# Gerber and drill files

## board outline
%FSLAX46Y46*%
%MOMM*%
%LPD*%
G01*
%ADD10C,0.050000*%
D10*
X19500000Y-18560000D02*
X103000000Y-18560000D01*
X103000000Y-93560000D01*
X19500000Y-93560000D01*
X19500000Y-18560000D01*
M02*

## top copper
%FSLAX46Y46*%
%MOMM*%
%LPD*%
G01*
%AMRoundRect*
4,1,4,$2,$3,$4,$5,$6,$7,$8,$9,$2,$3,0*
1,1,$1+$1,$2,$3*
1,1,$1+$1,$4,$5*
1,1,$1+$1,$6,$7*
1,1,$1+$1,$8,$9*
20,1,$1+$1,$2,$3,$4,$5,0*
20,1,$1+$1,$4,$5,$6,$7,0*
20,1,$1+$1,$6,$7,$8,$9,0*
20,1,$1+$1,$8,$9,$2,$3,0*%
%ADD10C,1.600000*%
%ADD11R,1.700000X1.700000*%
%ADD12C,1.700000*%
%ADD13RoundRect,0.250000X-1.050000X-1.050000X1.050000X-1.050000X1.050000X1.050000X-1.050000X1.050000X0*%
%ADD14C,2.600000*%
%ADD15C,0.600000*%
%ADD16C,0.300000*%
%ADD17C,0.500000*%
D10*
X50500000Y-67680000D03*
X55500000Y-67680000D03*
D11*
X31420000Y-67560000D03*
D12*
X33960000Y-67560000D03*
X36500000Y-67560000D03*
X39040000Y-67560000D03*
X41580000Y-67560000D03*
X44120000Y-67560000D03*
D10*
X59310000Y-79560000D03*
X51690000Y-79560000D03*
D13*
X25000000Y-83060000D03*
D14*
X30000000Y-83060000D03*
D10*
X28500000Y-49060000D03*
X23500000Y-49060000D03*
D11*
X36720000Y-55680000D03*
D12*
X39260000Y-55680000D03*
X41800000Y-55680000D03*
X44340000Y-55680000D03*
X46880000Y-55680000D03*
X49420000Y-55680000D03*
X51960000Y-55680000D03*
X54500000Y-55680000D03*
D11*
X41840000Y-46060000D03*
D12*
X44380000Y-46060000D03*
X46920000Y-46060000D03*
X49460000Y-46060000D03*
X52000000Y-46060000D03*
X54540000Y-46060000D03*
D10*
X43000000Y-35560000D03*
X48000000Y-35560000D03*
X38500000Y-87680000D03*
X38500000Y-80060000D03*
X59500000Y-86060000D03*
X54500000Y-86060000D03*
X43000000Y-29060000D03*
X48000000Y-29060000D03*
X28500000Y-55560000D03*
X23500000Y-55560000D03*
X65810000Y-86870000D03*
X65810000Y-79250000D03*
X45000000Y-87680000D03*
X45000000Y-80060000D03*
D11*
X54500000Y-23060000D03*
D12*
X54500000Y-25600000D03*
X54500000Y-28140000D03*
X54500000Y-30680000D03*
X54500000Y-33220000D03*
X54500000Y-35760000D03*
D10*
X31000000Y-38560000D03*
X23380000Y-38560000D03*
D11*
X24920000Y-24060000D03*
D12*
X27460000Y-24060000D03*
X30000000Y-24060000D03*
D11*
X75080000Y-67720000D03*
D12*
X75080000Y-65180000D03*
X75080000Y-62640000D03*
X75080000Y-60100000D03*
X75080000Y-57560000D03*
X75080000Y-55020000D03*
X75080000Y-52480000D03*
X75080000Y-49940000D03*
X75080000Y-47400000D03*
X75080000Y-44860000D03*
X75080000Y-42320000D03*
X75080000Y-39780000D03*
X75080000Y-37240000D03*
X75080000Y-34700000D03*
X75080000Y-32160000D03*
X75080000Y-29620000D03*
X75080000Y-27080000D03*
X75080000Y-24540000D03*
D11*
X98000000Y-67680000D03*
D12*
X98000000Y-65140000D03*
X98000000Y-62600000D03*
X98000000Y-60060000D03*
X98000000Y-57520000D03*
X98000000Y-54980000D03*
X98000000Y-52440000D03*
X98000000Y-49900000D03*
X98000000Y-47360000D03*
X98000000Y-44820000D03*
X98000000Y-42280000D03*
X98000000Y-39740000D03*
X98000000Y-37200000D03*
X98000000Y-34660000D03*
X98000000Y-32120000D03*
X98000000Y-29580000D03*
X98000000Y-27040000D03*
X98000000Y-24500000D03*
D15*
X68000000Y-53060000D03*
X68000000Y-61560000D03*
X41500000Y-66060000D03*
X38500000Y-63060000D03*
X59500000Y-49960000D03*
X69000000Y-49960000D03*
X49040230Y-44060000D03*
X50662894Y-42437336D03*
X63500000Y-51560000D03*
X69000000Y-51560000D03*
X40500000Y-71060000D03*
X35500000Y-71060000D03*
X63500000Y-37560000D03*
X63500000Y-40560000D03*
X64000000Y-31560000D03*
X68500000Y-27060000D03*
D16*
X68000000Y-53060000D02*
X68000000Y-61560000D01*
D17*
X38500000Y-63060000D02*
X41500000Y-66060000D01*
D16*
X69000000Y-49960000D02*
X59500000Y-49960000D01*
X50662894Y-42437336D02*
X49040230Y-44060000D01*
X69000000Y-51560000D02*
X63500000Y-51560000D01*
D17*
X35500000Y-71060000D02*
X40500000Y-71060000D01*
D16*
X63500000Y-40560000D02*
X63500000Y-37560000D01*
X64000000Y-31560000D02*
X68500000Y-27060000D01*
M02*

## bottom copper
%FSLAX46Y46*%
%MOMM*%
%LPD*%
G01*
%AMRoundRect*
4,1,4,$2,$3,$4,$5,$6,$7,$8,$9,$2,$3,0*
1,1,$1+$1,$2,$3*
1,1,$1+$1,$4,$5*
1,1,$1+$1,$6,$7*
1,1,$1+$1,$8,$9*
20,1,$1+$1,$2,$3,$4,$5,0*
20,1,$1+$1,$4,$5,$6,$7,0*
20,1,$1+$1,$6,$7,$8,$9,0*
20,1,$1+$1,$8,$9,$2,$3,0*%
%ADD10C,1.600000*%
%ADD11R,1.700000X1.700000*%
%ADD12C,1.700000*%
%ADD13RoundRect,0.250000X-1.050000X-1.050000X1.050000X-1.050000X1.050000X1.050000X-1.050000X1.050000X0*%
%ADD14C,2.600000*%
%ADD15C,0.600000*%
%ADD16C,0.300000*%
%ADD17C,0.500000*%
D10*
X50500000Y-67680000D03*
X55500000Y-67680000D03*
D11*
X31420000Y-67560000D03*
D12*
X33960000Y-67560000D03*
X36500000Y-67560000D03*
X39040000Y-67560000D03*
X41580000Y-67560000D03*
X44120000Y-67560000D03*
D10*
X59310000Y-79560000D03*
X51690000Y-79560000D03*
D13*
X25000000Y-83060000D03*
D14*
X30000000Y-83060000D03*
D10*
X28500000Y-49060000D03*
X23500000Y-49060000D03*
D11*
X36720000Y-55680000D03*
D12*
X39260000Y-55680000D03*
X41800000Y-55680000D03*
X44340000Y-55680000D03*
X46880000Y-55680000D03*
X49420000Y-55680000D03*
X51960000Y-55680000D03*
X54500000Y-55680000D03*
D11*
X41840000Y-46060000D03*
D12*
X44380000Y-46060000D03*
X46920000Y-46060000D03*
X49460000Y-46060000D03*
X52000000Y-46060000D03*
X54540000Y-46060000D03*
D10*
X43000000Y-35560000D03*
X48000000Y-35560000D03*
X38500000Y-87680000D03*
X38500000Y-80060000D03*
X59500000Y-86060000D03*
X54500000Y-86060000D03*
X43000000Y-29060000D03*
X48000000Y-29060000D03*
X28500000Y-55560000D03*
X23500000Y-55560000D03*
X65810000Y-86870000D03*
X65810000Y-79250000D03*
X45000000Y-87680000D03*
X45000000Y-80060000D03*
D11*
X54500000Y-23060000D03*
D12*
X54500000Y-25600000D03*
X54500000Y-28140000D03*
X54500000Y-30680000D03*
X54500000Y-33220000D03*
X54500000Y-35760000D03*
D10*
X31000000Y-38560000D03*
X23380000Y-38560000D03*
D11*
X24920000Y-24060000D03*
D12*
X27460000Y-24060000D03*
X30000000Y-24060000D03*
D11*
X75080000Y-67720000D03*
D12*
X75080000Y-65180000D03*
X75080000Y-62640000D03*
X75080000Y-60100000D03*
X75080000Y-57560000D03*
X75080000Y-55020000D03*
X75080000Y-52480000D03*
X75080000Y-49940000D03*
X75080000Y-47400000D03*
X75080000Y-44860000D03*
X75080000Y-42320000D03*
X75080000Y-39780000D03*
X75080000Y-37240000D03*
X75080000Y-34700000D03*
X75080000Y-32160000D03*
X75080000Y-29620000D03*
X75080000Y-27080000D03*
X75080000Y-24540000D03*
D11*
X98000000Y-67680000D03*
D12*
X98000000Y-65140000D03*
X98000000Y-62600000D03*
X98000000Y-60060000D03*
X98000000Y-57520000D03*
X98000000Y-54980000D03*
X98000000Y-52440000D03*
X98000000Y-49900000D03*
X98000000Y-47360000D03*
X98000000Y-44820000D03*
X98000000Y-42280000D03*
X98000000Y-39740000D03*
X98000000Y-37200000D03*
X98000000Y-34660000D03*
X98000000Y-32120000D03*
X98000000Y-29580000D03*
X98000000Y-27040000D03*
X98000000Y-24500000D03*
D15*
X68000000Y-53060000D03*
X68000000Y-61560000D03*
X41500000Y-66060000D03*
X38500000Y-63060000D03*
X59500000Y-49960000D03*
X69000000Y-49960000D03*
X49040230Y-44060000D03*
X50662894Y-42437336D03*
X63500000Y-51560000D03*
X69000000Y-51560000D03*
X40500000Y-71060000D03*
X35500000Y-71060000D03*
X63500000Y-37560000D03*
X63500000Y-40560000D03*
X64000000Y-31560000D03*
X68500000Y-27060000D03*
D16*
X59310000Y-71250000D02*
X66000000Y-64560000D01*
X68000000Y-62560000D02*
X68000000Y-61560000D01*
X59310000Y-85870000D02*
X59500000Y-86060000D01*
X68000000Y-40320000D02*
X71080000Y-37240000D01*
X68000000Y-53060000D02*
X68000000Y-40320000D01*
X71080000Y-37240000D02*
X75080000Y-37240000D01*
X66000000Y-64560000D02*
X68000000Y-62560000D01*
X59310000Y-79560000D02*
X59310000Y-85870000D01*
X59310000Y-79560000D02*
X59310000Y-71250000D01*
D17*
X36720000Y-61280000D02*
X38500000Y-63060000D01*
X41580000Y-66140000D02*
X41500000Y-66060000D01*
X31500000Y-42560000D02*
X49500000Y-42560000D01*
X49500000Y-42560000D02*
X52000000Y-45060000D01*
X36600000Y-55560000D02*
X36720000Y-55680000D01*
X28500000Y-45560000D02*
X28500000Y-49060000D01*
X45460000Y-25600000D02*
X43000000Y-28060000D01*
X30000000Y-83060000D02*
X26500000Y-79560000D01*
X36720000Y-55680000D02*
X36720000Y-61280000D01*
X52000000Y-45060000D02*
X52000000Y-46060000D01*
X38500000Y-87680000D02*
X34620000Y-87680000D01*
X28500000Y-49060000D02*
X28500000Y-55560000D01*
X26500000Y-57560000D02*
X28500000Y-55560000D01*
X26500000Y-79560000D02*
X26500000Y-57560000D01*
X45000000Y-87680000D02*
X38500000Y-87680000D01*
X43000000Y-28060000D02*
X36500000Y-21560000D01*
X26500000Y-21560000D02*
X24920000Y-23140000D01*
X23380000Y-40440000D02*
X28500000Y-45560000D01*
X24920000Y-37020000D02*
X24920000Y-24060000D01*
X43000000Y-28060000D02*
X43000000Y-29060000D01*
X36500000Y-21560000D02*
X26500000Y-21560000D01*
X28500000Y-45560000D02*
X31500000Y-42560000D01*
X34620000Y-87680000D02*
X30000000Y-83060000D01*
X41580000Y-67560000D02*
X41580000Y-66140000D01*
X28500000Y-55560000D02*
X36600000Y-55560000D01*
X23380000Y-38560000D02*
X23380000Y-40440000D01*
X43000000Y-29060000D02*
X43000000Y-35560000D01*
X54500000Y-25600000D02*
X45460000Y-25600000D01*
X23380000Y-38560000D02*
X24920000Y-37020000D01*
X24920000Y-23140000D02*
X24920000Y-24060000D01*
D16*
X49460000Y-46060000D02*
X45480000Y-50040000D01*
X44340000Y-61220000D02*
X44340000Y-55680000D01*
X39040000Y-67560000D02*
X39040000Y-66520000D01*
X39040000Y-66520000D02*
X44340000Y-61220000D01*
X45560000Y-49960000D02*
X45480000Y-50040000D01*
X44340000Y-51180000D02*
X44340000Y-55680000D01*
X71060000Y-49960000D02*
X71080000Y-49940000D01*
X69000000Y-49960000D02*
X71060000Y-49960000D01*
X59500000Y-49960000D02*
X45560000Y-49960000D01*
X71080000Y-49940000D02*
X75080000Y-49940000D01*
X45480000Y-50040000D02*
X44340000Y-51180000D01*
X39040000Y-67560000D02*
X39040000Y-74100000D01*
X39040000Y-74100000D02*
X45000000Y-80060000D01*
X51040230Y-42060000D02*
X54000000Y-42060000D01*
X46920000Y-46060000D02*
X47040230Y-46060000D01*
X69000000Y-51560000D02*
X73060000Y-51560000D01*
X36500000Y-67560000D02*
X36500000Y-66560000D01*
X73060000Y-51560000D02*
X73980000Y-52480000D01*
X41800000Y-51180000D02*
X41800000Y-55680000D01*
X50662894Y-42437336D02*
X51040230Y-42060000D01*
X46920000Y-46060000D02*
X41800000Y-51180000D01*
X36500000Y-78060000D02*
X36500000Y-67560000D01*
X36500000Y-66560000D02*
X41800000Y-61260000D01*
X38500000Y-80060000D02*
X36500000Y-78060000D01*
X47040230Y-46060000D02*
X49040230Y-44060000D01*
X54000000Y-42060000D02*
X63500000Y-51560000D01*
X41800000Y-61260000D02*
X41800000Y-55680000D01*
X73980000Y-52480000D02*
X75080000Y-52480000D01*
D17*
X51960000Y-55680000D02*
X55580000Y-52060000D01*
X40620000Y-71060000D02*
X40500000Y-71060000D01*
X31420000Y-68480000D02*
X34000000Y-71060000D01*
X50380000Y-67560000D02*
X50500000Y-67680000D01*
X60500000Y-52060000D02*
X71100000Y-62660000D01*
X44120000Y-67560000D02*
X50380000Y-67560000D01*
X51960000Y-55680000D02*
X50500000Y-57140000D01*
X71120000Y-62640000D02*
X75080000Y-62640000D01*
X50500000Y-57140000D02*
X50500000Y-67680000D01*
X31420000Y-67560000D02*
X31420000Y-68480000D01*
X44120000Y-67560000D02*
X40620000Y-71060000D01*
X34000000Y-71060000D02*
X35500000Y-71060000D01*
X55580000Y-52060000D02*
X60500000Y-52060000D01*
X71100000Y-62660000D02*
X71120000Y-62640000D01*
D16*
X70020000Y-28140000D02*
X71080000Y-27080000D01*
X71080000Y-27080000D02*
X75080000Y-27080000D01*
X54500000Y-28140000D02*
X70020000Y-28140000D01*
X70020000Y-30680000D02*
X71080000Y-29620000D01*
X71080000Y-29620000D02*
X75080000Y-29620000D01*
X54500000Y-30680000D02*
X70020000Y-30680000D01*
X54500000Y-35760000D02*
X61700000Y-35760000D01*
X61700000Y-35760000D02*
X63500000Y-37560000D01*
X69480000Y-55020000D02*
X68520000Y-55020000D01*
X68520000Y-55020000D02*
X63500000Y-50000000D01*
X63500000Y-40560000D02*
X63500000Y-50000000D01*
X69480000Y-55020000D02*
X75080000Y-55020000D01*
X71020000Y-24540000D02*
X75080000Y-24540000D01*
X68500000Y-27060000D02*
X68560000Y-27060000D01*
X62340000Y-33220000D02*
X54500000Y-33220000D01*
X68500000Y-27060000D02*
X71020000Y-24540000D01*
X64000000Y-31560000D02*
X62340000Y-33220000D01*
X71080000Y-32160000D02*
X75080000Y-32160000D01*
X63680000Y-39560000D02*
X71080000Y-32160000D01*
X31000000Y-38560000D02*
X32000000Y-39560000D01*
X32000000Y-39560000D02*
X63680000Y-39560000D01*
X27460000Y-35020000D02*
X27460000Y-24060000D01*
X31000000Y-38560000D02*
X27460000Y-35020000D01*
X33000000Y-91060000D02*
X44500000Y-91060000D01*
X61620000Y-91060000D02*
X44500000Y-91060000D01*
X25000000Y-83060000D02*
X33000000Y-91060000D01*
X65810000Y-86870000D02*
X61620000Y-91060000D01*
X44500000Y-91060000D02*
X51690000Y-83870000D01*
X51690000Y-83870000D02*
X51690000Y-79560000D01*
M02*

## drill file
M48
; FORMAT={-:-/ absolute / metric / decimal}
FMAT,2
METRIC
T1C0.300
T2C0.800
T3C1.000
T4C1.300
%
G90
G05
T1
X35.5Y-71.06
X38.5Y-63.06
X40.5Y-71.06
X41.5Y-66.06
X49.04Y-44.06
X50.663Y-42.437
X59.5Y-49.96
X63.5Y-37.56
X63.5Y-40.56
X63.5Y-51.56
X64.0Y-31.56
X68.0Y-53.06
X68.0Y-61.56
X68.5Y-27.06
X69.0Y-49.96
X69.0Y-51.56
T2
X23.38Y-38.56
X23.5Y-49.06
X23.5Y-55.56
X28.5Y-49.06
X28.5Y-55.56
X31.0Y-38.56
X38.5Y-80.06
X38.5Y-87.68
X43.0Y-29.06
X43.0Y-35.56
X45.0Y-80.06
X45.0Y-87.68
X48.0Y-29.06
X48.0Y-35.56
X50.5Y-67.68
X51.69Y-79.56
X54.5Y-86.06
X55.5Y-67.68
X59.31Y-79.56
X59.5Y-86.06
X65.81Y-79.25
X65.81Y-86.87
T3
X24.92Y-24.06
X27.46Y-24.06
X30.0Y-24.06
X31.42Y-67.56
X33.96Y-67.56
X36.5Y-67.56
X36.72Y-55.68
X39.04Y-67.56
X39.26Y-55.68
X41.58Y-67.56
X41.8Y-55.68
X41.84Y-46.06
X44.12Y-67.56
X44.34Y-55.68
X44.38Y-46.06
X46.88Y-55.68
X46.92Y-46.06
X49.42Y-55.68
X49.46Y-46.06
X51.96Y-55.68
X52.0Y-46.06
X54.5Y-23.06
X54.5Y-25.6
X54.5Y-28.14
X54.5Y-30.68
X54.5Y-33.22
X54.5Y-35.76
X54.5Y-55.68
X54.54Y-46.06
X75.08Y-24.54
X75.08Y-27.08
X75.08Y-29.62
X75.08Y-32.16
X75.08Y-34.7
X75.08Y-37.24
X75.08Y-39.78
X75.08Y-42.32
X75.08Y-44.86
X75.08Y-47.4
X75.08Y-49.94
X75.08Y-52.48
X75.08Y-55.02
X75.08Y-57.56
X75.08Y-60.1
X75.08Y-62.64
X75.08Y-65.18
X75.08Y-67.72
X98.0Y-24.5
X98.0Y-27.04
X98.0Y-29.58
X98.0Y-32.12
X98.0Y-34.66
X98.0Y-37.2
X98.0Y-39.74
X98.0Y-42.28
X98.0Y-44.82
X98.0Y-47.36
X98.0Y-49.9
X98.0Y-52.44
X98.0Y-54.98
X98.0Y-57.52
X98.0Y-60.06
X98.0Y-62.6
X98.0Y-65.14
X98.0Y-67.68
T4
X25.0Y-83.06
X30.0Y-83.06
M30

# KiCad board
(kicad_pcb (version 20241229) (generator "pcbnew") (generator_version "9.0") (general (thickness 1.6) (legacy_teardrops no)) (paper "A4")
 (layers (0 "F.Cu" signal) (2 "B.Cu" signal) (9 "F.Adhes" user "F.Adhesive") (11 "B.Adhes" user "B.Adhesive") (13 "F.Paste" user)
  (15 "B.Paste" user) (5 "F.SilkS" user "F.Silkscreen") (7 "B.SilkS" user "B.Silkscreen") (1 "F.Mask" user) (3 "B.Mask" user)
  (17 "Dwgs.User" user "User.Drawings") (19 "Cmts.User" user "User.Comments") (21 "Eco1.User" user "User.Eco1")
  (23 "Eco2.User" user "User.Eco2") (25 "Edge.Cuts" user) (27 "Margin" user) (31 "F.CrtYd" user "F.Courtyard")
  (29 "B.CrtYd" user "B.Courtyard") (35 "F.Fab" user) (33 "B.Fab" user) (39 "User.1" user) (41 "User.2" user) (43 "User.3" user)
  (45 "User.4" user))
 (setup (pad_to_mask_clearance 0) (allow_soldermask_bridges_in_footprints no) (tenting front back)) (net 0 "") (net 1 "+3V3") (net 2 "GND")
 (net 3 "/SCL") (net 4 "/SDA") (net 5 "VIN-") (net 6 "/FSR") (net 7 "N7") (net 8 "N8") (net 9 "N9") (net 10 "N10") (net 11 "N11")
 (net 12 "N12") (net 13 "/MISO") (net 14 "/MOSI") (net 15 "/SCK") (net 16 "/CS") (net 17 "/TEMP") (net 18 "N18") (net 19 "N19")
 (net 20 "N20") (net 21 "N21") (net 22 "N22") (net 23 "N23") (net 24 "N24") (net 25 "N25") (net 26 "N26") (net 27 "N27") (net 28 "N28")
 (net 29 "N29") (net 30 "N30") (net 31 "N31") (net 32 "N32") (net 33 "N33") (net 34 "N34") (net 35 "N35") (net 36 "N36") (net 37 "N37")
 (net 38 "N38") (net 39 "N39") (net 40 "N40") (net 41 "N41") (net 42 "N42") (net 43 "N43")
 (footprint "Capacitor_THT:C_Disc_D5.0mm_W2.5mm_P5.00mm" (layer "F.Cu") (at 50.5 67.68)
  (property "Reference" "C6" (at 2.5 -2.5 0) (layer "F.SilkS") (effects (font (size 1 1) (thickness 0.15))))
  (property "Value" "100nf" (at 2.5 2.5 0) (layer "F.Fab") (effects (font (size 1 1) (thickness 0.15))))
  (pad "1" thru_hole circle (at 0 0) (size 1.6 1.6) (drill 0.8) (layers "*.Cu" "*.Mask") (remove_unused_layers no) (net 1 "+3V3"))
  (pad "2" thru_hole circle (at 5 0) (size 1.6 1.6) (drill 0.8) (layers "*.Cu" "*.Mask") (remove_unused_layers no) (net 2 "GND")))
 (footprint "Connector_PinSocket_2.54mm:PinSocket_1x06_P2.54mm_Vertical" (layer "F.Cu") (at 31.42 67.56 90)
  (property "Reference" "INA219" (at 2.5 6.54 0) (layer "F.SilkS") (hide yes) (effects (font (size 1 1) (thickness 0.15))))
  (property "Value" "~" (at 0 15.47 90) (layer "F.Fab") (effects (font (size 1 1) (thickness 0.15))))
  (pad "1" thru_hole rect (at 0 0 90) (size 1.7 1.7) (drill 1) (layers "*.Cu" "*.Mask") (remove_unused_layers no) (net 1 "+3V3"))
  (pad "2" thru_hole circle (at 0 2.54 90) (size 1.7 1.7) (drill 1) (layers "*.Cu" "*.Mask") (remove_unused_layers no) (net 2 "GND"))
  (pad "3" thru_hole circle (at 0 5.08 90) (size 1.7 1.7) (drill 1) (layers "*.Cu" "*.Mask") (remove_unused_layers no) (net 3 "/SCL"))
  (pad "4" thru_hole circle (at 0 7.62 90) (size 1.7 1.7) (drill 1) (layers "*.Cu" "*.Mask") (remove_unused_layers no) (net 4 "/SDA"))
  (pad "5" thru_hole circle (at 0 10.16 90) (size 1.7 1.7) (drill 1) (layers "*.Cu" "*.Mask") (remove_unused_layers no) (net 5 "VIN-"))
  (pad "6" thru_hole circle (at 0 12.7 90) (size 1.7 1.7) (drill 1) (layers "*.Cu" "*.Mask") (remove_unused_layers no) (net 1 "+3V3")))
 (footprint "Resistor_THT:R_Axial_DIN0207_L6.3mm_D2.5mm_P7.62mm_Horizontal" (layer "F.Cu") (at 59.31 79.56 180)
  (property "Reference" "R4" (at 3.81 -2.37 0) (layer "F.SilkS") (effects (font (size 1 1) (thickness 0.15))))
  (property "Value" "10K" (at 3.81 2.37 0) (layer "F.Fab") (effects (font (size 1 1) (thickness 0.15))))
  (pad "1" thru_hole circle (at 0 0 180) (size 1.6 1.6) (drill 0.8) (layers "*.Cu" "*.Mask") (remove_unused_layers no) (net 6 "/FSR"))
  (pad "2" thru_hole circle (at 7.62 0 180) (size 1.6 1.6) (drill 0.8) (layers "*.Cu" "*.Mask") (remove_unused_layers no) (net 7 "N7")))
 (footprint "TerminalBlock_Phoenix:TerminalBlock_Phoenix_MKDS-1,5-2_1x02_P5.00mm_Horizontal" (layer "F.Cu") (at 25 83.06)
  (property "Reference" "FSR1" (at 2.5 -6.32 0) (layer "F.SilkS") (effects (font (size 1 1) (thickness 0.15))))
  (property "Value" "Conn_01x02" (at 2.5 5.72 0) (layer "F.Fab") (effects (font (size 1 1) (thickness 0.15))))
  (pad "1" thru_hole roundrect (at 0 0) (size 2.6 2.6) (drill 1.3) (layers "*.Cu" "*.Mask") (remove_unused_layers no)
   (roundrect_rratio 0.096154) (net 7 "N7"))
  (pad "2" thru_hole circle (at 5 0) (size 2.6 2.6) (drill 1.3) (layers "*.Cu" "*.Mask") (remove_unused_layers no) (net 5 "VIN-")))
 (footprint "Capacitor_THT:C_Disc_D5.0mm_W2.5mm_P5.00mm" (layer "F.Cu") (at 28.5 49.06 180)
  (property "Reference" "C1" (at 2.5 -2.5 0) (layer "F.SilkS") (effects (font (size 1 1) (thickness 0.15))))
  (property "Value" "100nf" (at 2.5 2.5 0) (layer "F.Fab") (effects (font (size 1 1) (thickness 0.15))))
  (pad "1" thru_hole circle (at 0 0 180) (size 1.6 1.6) (drill 0.8) (layers "*.Cu" "*.Mask") (remove_unused_layers no) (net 5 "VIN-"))
  (pad "2" thru_hole circle (at 5 0 180) (size 1.6 1.6) (drill 0.8) (layers "*.Cu" "*.Mask") (remove_unused_layers no) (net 2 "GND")))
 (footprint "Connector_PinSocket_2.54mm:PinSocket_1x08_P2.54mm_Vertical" (layer "F.Cu") (at 36.72 55.68 90)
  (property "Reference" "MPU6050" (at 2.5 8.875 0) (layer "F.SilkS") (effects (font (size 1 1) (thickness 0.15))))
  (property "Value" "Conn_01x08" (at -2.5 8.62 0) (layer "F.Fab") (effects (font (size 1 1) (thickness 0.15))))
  (pad "1" thru_hole rect (at 0 0 90) (size 1.7 1.7) (drill 1) (layers "*.Cu" "*.Mask") (remove_unused_layers no) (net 5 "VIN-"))
  (pad "2" thru_hole circle (at 0 2.54 90) (size 1.7 1.7) (drill 1) (layers "*.Cu" "*.Mask") (remove_unused_layers no) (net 2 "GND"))
  (pad "3" thru_hole circle (at 0 5.08 90) (size 1.7 1.7) (drill 1) (layers "*.Cu" "*.Mask") (remove_unused_layers no) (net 3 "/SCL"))
  (pad "4" thru_hole circle (at 0 7.62 90) (size 1.7 1.7) (drill 1) (layers "*.Cu" "*.Mask") (remove_unused_layers no) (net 4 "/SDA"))
  (pad "5" thru_hole circle (at 0 10.16 90) (size 1.7 1.7) (drill 1) (layers "*.Cu" "*.Mask") (remove_unused_layers no) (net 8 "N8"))
  (pad "6" thru_hole circle (at 0 12.7 90) (size 1.7 1.7) (drill 1) (layers "*.Cu" "*.Mask") (remove_unused_layers no) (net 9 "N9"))
  (pad "7" thru_hole circle (at 0 15.24 90) (size 1.7 1.7) (drill 1) (layers "*.Cu" "*.Mask") (remove_unused_layers no) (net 1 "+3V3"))
  (pad "8" thru_hole circle (at 0 17.78 90) (size 1.7 1.7) (drill 1) (layers "*.Cu" "*.Mask") (remove_unused_layers no) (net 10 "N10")))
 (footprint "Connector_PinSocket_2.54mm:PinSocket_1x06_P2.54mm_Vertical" (layer "F.Cu") (at 41.84 46.06 90)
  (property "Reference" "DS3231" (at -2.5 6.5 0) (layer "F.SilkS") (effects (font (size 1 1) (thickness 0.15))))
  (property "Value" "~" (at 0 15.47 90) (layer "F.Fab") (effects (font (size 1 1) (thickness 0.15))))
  (pad "1" thru_hole rect (at 0 0 90) (size 1.7 1.7) (drill 1) (layers "*.Cu" "*.Mask") (remove_unused_layers no) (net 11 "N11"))
  (pad "2" thru_hole circle (at 0 2.54 90) (size 1.7 1.7) (drill 1) (layers "*.Cu" "*.Mask") (remove_unused_layers no) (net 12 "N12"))
  (pad "3" thru_hole circle (at 0 5.08 90) (size 1.7 1.7) (drill 1) (layers "*.Cu" "*.Mask") (remove_unused_layers no) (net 3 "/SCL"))
  (pad "4" thru_hole circle (at 0 7.62 90) (size 1.7 1.7) (drill 1) (layers "*.Cu" "*.Mask") (remove_unused_layers no) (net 4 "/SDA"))
  (pad "5" thru_hole circle (at 0 10.16 90) (size 1.7 1.7) (drill 1) (layers "*.Cu" "*.Mask") (remove_unused_layers no) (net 5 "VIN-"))
  (pad "6" thru_hole circle (at 0 12.7 90) (size 1.7 1.7) (drill 1) (layers "*.Cu" "*.Mask") (remove_unused_layers no) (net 2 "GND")))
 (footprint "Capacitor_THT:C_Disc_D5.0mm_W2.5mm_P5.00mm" (layer "F.Cu") (at 43 35.56)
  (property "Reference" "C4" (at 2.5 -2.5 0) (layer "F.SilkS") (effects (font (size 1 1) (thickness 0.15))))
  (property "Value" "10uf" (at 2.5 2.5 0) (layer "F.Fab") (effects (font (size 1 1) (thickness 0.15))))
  (pad "1" thru_hole circle (at 0 0) (size 1.6 1.6) (drill 0.8) (layers "*.Cu" "*.Mask") (remove_unused_layers no) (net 5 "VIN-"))
  (pad "2" thru_hole circle (at 5 0) (size 1.6 1.6) (drill 0.8) (layers "*.Cu" "*.Mask") (remove_unused_layers no) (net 2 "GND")))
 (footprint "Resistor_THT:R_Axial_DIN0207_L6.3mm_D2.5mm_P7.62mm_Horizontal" (layer "F.Cu") (at 38.5 87.68 90)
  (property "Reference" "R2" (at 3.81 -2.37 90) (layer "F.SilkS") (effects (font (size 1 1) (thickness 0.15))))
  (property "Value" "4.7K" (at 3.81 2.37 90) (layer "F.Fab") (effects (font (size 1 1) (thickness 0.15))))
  (pad "1" thru_hole circle (at 0 0 90) (size 1.6 1.6) (drill 0.8) (layers "*.Cu" "*.Mask") (remove_unused_layers no) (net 5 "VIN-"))
  (pad "2" thru_hole circle (at 7.62 0 90) (size 1.6 1.6) (drill 0.8) (layers "*.Cu" "*.Mask") (remove_unused_layers no) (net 3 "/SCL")))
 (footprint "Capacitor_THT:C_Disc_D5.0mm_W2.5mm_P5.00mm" (layer "F.Cu") (at 59.5 86.06 180)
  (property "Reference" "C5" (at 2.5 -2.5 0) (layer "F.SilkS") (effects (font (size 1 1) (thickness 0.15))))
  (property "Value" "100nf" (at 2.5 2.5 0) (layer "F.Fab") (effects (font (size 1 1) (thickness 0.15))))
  (pad "1" thru_hole circle (at 0 0 180) (size 1.6 1.6) (drill 0.8) (layers "*.Cu" "*.Mask") (remove_unused_layers no) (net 6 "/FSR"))
  (pad "2" thru_hole circle (at 5 0 180) (size 1.6 1.6) (drill 0.8) (layers "*.Cu" "*.Mask") (remove_unused_layers no) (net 2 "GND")))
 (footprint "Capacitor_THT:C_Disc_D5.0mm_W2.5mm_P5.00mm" (layer "F.Cu") (at 43 29.06)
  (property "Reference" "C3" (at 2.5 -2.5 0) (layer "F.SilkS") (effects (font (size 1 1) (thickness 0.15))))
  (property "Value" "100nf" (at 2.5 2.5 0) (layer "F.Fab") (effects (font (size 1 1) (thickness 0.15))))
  (pad "1" thru_hole circle (at 0 0) (size 1.6 1.6) (drill 0.8) (layers "*.Cu" "*.Mask") (remove_unused_layers no) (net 5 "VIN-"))
  (pad "2" thru_hole circle (at 5 0) (size 1.6 1.6) (drill 0.8) (layers "*.Cu" "*.Mask") (remove_unused_layers no) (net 2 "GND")))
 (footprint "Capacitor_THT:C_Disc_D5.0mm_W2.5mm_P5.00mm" (layer "F.Cu") (at 28.5 55.56 180)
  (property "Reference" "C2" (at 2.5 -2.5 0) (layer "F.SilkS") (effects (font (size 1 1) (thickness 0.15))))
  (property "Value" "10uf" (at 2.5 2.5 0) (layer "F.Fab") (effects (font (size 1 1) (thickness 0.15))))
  (pad "1" thru_hole circle (at 0 0 180) (size 1.6 1.6) (drill 0.8) (layers "*.Cu" "*.Mask") (remove_unused_layers no) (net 5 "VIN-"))
  (pad "2" thru_hole circle (at 5 0 180) (size 1.6 1.6) (drill 0.8) (layers "*.Cu" "*.Mask") (remove_unused_layers no) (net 2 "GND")))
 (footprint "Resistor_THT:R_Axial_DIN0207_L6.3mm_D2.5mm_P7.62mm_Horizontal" (layer "F.Cu") (at 65.81 86.87 90)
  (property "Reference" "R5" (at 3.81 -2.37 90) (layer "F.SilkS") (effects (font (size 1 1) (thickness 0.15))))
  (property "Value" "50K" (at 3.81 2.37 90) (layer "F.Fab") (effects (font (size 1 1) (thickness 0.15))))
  (pad "1" thru_hole circle (at 0 0 90) (size 1.6 1.6) (drill 0.8) (layers "*.Cu" "*.Mask") (remove_unused_layers no) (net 7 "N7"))
  (pad "2" thru_hole circle (at 7.62 0 90) (size 1.6 1.6) (drill 0.8) (layers "*.Cu" "*.Mask") (remove_unused_layers no) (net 2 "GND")))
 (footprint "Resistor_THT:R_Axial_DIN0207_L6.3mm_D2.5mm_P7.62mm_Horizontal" (layer "F.Cu") (at 45 87.68 90)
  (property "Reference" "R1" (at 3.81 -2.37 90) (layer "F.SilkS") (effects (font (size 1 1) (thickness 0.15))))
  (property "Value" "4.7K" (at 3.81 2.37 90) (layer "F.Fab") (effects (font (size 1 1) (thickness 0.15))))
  (pad "1" thru_hole circle (at 0 0 90) (size 1.6 1.6) (drill 0.8) (layers "*.Cu" "*.Mask") (remove_unused_layers no) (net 5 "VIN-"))
  (pad "2" thru_hole circle (at 7.62 0 90) (size 1.6 1.6) (drill 0.8) (layers "*.Cu" "*.Mask") (remove_unused_layers no) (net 4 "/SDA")))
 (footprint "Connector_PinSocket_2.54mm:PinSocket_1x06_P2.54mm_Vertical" (layer "F.Cu") (at 54.5 23.06)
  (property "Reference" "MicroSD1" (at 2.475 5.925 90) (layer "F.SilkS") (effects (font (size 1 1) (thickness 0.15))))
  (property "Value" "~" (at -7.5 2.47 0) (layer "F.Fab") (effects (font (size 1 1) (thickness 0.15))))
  (pad "1" thru_hole rect (at 0 0) (size 1.7 1.7) (drill 1) (layers "*.Cu" "*.Mask") (remove_unused_layers no) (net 2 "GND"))
  (pad "2" thru_hole circle (at 0 2.54) (size 1.7 1.7) (drill 1) (layers "*.Cu" "*.Mask") (remove_unused_layers no) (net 5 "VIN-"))
  (pad "3" thru_hole circle (at 0 5.08) (size 1.7 1.7) (drill 1) (layers "*.Cu" "*.Mask") (remove_unused_layers no) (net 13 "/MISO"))
  (pad "4" thru_hole circle (at 0 7.62) (size 1.7 1.7) (drill 1) (layers "*.Cu" "*.Mask") (remove_unused_layers no) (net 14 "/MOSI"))
  (pad "5" thru_hole circle (at 0 10.16) (size 1.7 1.7) (drill 1) (layers "*.Cu" "*.Mask") (remove_unused_layers no) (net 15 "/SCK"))
  (pad "6" thru_hole circle (at 0 12.7) (size 1.7 1.7) (drill 1) (layers "*.Cu" "*.Mask") (remove_unused_layers no) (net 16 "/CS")))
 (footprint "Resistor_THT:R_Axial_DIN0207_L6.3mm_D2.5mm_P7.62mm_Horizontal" (layer "F.Cu") (at 31 38.56 180)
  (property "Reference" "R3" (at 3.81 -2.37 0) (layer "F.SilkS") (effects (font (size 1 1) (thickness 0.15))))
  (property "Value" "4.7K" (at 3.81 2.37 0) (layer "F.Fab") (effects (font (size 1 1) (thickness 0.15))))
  (pad "1" thru_hole circle (at 0 0 180) (size 1.6 1.6) (drill 0.8) (layers "*.Cu" "*.Mask") (remove_unused_layers no) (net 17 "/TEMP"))
  (pad "2" thru_hole circle (at 7.62 0 180) (size 1.6 1.6) (drill 0.8) (layers "*.Cu" "*.Mask") (remove_unused_layers no) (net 5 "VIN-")))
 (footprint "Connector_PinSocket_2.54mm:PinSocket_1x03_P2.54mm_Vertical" (layer "F.Cu") (at 24.92 24.06 90)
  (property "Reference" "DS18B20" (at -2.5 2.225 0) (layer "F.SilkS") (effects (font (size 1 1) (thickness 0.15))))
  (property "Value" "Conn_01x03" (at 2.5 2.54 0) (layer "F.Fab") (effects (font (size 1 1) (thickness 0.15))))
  (pad "1" thru_hole rect (at 0 0 90) (size 1.7 1.7) (drill 1) (layers "*.Cu" "*.Mask") (remove_unused_layers no) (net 5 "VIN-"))
  (pad "2" thru_hole circle (at 0 2.54 90) (size 1.7 1.7) (drill 1) (layers "*.Cu" "*.Mask") (remove_unused_layers no) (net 17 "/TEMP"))
  (pad "3" thru_hole circle (at 0 5.08 90) (size 1.7 1.7) (drill 1) (layers "*.Cu" "*.Mask") (remove_unused_layers no) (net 2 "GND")))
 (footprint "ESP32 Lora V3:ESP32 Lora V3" (layer "F.Cu") (at 86.58 46.41)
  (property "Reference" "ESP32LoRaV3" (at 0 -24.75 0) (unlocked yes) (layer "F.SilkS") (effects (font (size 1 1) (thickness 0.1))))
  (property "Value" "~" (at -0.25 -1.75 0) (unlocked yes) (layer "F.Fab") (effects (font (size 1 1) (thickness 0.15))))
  (pad "1" thru_hole rect (at -11.5 21.31 180) (size 1.7 1.7) (drill 1) (layers "*.Cu" "*.Mask") (remove_unused_layers no) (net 2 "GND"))
  (pad "2" thru_hole circle (at -11.5 18.77 180) (size 1.7 1.7) (drill 1) (layers "*.Cu" "*.Mask") (remove_unused_layers no) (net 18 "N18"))
  (pad "3" thru_hole circle (at -11.5 16.23 180) (size 1.7 1.7) (drill 1) (layers "*.Cu" "*.Mask") (remove_unused_layers no) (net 1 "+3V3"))
  (pad "4" thru_hole circle (at -11.5 13.69 180) (size 1.7 1.7) (drill 1) (layers "*.Cu" "*.Mask") (remove_unused_layers no) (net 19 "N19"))
  (pad "5" thru_hole circle (at -11.5 11.15 180) (size 1.7 1.7) (drill 1) (layers "*.Cu" "*.Mask") (remove_unused_layers no) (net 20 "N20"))
  (pad "6" thru_hole circle (at -11.5 8.61 180) (size 1.7 1.7) (drill 1) (layers "*.Cu" "*.Mask") (remove_unused_layers no) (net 16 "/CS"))
  (pad "7" thru_hole circle (at -11.5 6.07 180) (size 1.7 1.7) (drill 1) (layers "*.Cu" "*.Mask") (remove_unused_layers no) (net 3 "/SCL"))
  (pad "8" thru_hole circle (at -11.5 3.53 180) (size 1.7 1.7) (drill 1) (layers "*.Cu" "*.Mask") (remove_unused_layers no) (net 4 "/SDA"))
  (pad "9" thru_hole circle (at -11.5 0.99 180) (size 1.7 1.7) (drill 1) (layers "*.Cu" "*.Mask") (remove_unused_layers no) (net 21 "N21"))
  (pad "10" thru_hole circle (at -11.5 -1.55 180) (size 1.7 1.7) (drill 1) (layers "*.Cu" "*.Mask") (remove_unused_layers no) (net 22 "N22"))
  (pad "11" thru_hole circle (at -11.5 -4.09 180) (size 1.7 1.7) (drill 1) (layers "*.Cu" "*.Mask") (remove_unused_layers no) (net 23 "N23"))
  (pad "12" thru_hole circle (at -11.5 -6.63 180) (size 1.7 1.7) (drill 1) (layers "*.Cu" "*.Mask") (remove_unused_layers no) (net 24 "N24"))
  (pad "13" thru_hole circle (at -11.5 -9.17 180) (size 1.7 1.7) (drill 1) (layers "*.Cu" "*.Mask") (remove_unused_layers no) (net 6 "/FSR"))
  (pad "14" thru_hole circle (at -11.5 -11.71 180) (size 1.7 1.7) (drill 1) (layers "*.Cu" "*.Mask") (remove_unused_layers no)
   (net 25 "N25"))
  (pad "15" thru_hole circle (at -11.5 -14.25 180) (size 1.7 1.7) (drill 1) (layers "*.Cu" "*.Mask") (remove_unused_layers no)
   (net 17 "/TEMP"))
  (pad "16" thru_hole circle (at -11.5 -16.79 180) (size 1.7 1.7) (drill 1) (layers "*.Cu" "*.Mask") (remove_unused_layers no)
   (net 14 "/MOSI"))
  (pad "17" thru_hole circle (at -11.5 -19.33 180) (size 1.7 1.7) (drill 1) (layers "*.Cu" "*.Mask") (remove_unused_layers no)
   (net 13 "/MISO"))
  (pad "18" thru_hole circle (at -11.5 -21.87 180) (size 1.7 1.7) (drill 1) (layers "*.Cu" "*.Mask") (remove_unused_layers no)
   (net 15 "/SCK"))
  (pad "19" thru_hole rect (at 11.42 21.27 180) (size 1.7 1.7) (drill 1) (layers "*.Cu" "*.Mask") (remove_unused_layers no) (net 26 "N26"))
  (pad "20" thru_hole circle (at 11.42 18.73 180) (size 1.7 1.7) (drill 1) (layers "*.Cu" "*.Mask") (remove_unused_layers no) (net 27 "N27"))
  (pad "21" thru_hole circle (at 11.42 16.19 180) (size 1.7 1.7) (drill 1) (layers "*.Cu" "*.Mask") (remove_unused_layers no) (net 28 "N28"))
  (pad "22" thru_hole circle (at 11.42 13.65 180) (size 1.7 1.7) (drill 1) (layers "*.Cu" "*.Mask") (remove_unused_layers no) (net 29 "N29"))
  (pad "23" thru_hole circle (at 11.42 11.11 180) (size 1.7 1.7) (drill 1) (layers "*.Cu" "*.Mask") (remove_unused_layers no) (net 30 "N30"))
  (pad "24" thru_hole circle (at 11.42 8.57 180) (size 1.7 1.7) (drill 1) (layers "*.Cu" "*.Mask") (remove_unused_layers no) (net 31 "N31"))
  (pad "25" thru_hole circle (at 11.42 6.03 180) (size 1.7 1.7) (drill 1) (layers "*.Cu" "*.Mask") (remove_unused_layers no) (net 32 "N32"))
  (pad "26" thru_hole circle (at 11.42 3.49 180) (size 1.7 1.7) (drill 1) (layers "*.Cu" "*.Mask") (remove_unused_layers no) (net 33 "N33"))
  (pad "27" thru_hole circle (at 11.42 0.95 180) (size 1.7 1.7) (drill 1) (layers "*.Cu" "*.Mask") (remove_unused_layers no) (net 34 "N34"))
  (pad "28" thru_hole circle (at 11.42 -1.59 180) (size 1.7 1.7) (drill 1) (layers "*.Cu" "*.Mask") (remove_unused_layers no) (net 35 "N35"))
  (pad "29" thru_hole circle (at 11.42 -4.13 180) (size 1.7 1.7) (drill 1) (layers "*.Cu" "*.Mask") (remove_unused_layers no) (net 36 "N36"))
  (pad "30" thru_hole circle (at 11.42 -6.67 180) (size 1.7 1.7) (drill 1) (layers "*.Cu" "*.Mask") (remove_unused_layers no) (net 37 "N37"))
  (pad "31" thru_hole circle (at 11.42 -9.21 180) (size 1.7 1.7) (drill 1) (layers "*.Cu" "*.Mask") (remove_unused_layers no) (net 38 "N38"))
  (pad "32" thru_hole circle (at 11.42 -11.75 180) (size 1.7 1.7) (drill 1) (layers "*.Cu" "*.Mask") (remove_unused_layers no)
   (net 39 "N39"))
  (pad "33" thru_hole circle (at 11.42 -14.29 180) (size 1.7 1.7) (drill 1) (layers "*.Cu" "*.Mask") (remove_unused_layers no)
   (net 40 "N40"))
  (pad "34" thru_hole circle (at 11.42 -16.83 180) (size 1.7 1.7) (drill 1) (layers "*.Cu" "*.Mask") (remove_unused_layers no)
   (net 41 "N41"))
  (pad "35" thru_hole circle (at 11.42 -19.37 180) (size 1.7 1.7) (drill 1) (layers "*.Cu" "*.Mask") (remove_unused_layers no)
   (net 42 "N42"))
  (pad "36" thru_hole circle (at 11.42 -21.91 180) (size 1.7 1.7) (drill 1) (layers "*.Cu" "*.Mask") (remove_unused_layers no)
   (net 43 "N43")))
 (gr_rect (start 19.5 18.56) (end 103 93.56) (stroke (width 0.05) (type solid)) (fill no) (layer "Edge.Cuts"))
 (segment (start 68 53.06) (end 68 61.56) (width 0.3) (layer "F.Cu") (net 6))
 (via (at 68 53.06) (size 0.6) (drill 0.3) (layers "F.Cu" "B.Cu") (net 6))
 (via (at 68 61.56) (size 0.6) (drill 0.3) (layers "F.Cu" "B.Cu") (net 6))
 (segment (start 59.31 71.25) (end 66 64.56) (width 0.3) (layer "B.Cu") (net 6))
 (segment (start 68 62.56) (end 68 61.56) (width 0.3) (layer "B.Cu") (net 6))
 (segment (start 59.31 85.87) (end 59.5 86.06) (width 0.3) (layer "B.Cu") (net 6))
 (segment (start 68 40.32) (end 71.08 37.24) (width 0.3) (layer "B.Cu") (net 6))
 (segment (start 68 53.06) (end 68 40.32) (width 0.3) (layer "B.Cu") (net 6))
 (segment (start 71.08 37.24) (end 75.08 37.24) (width 0.3) (layer "B.Cu") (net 6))
 (segment (start 66 64.56) (end 68 62.56) (width 0.3) (layer "B.Cu") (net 6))
 (segment (start 59.31 79.56) (end 59.31 85.87) (width 0.3) (layer "B.Cu") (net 6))
 (segment (start 59.31 79.56) (end 59.31 71.25) (width 0.3) (layer "B.Cu") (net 6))
 (segment (start 38.5 63.06) (end 41.5 66.06) (width 0.5) (layer "F.Cu") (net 5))
 (via (at 41.5 66.06) (size 0.6) (drill 0.3) (layers "F.Cu" "B.Cu") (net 5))
 (via (at 38.5 63.06) (size 0.6) (drill 0.3) (layers "F.Cu" "B.Cu") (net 5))
 (segment (start 36.72 61.28) (end 38.5 63.06) (width 0.5) (layer "B.Cu") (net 5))
 (segment (start 41.58 66.14) (end 41.5 66.06) (width 0.5) (layer "B.Cu") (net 5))
 (segment (start 31.5 42.56) (end 49.5 42.56) (width 0.5) (layer "B.Cu") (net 5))
 (segment (start 49.5 42.56) (end 52 45.06) (width 0.5) (layer "B.Cu") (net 5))
 (segment (start 36.6 55.56) (end 36.72 55.68) (width 0.5) (layer "B.Cu") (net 5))
 (segment (start 28.5 45.56) (end 28.5 49.06) (width 0.5) (layer "B.Cu") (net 5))
 (segment (start 45.46 25.6) (end 43 28.06) (width 0.5) (layer "B.Cu") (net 5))
 (segment (start 30 83.06) (end 26.5 79.56) (width 0.5) (layer "B.Cu") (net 5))
 (segment (start 36.72 55.68) (end 36.72 61.28) (width 0.5) (layer "B.Cu") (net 5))
 (segment (start 52 45.06) (end 52 46.06) (width 0.5) (layer "B.Cu") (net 5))
 (segment (start 38.5 87.68) (end 34.62 87.68) (width 0.5) (layer "B.Cu") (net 5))
 (segment (start 28.5 49.06) (end 28.5 55.56) (width 0.5) (layer "B.Cu") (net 5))
 (segment (start 26.5 57.56) (end 28.5 55.56) (width 0.5) (layer "B.Cu") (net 5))
 (segment (start 26.5 79.56) (end 26.5 57.56) (width 0.5) (layer "B.Cu") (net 5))
 (segment (start 45 87.68) (end 38.5 87.68) (width 0.5) (layer "B.Cu") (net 5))
 (segment (start 43 28.06) (end 36.5 21.56) (width 0.5) (layer "B.Cu") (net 5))
 (segment (start 26.5 21.56) (end 24.92 23.14) (width 0.5) (layer "B.Cu") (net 5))
 (segment (start 23.38 40.44) (end 28.5 45.56) (width 0.5) (layer "B.Cu") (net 5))
 (segment (start 24.92 37.02) (end 24.92 24.06) (width 0.5) (layer "B.Cu") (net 5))
 (segment (start 43 28.06) (end 43 29.06) (width 0.5) (layer "B.Cu") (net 5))
 (segment (start 36.5 21.56) (end 26.5 21.56) (width 0.5) (layer "B.Cu") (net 5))
 (segment (start 28.5 45.56) (end 31.5 42.56) (width 0.5) (layer "B.Cu") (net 5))
 (segment (start 34.62 87.68) (end 30 83.06) (width 0.5) (layer "B.Cu") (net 5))
 (segment (start 41.58 67.56) (end 41.58 66.14) (width 0.5) (layer "B.Cu") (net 5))
 (segment (start 28.5 55.56) (end 36.6 55.56) (width 0.5) (layer "B.Cu") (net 5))
 (segment (start 23.38 38.56) (end 23.38 40.44) (width 0.5) (layer "B.Cu") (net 5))
 (segment (start 43 29.06) (end 43 35.56) (width 0.5) (layer "B.Cu") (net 5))
 (segment (start 54.5 25.6) (end 45.46 25.6) (width 0.5) (layer "B.Cu") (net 5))
 (segment (start 23.38 38.56) (end 24.92 37.02) (width 0.5) (layer "B.Cu") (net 5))
 (segment (start 24.92 23.14) (end 24.92 24.06) (width 0.5) (layer "B.Cu") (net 5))
 (segment (start 69 49.96) (end 59.5 49.96) (width 0.3) (layer "F.Cu") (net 4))
 (via (at 59.5 49.96) (size 0.6) (drill 0.3) (layers "F.Cu" "B.Cu") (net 4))
 (via (at 69 49.96) (size 0.6) (drill 0.3) (layers "F.Cu" "B.Cu") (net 4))
 (segment (start 49.46 46.06) (end 45.48 50.04) (width 0.3) (layer "B.Cu") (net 4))
 (segment (start 44.34 61.22) (end 44.34 55.68) (width 0.3) (layer "B.Cu") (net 4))
 (segment (start 39.04 67.56) (end 39.04 66.52) (width 0.3) (layer "B.Cu") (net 4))
 (segment (start 39.04 66.52) (end 44.34 61.22) (width 0.3) (layer "B.Cu") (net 4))
 (segment (start 45.56 49.96) (end 45.48 50.04) (width 0.3) (layer "B.Cu") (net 4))
 (segment (start 44.34 51.18) (end 44.34 55.68) (width 0.3) (layer "B.Cu") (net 4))
 (segment (start 71.06 49.96) (end 71.08 49.94) (width 0.3) (layer "B.Cu") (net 4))
 (segment (start 69 49.96) (end 71.06 49.96) (width 0.3) (layer "B.Cu") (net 4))
 (segment (start 59.5 49.96) (end 45.56 49.96) (width 0.3) (layer "B.Cu") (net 4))
 (segment (start 71.08 49.94) (end 75.08 49.94) (width 0.3) (layer "B.Cu") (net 4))
 (segment (start 45.48 50.04) (end 44.34 51.18) (width 0.3) (layer "B.Cu") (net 4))
 (segment (start 39.04 67.56) (end 39.04 74.1) (width 0.3) (layer "B.Cu") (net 4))
 (segment (start 39.04 74.1) (end 45 80.06) (width 0.3) (layer "B.Cu") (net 4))
 (segment (start 50.662894 42.437336) (end 49.04023 44.06) (width 0.3) (layer "F.Cu") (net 3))
 (segment (start 69 51.56) (end 63.5 51.56) (width 0.3) (layer "F.Cu") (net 3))
 (via (at 49.04023 44.06) (size 0.6) (drill 0.3) (layers "F.Cu" "B.Cu") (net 3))
 (via (at 50.662894 42.437336) (size 0.6) (drill 0.3) (layers "F.Cu" "B.Cu") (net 3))
 (via (at 63.5 51.56) (size 0.6) (drill 0.3) (layers "F.Cu" "B.Cu") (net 3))
 (via (at 69 51.56) (size 0.6) (drill 0.3) (layers "F.Cu" "B.Cu") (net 3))
 (segment (start 51.04023 42.06) (end 54 42.06) (width 0.3) (layer "B.Cu") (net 3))
 (segment (start 46.92 46.06) (end 47.04023 46.06) (width 0.3) (layer "B.Cu") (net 3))
 (segment (start 69 51.56) (end 73.06 51.56) (width 0.3) (layer "B.Cu") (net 3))
 (segment (start 36.5 67.56) (end 36.5 66.56) (width 0.3) (layer "B.Cu") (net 3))
 (segment (start 73.06 51.56) (end 73.98 52.48) (width 0.3) (layer "B.Cu") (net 3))
 (segment (start 41.8 51.18) (end 41.8 55.68) (width 0.3) (layer "B.Cu") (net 3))
 (segment (start 50.662894 42.437336) (end 51.04023 42.06) (width 0.3) (layer "B.Cu") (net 3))
 (segment (start 46.92 46.06) (end 41.8 51.18) (width 0.3) (layer "B.Cu") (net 3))
 (segment (start 36.5 78.06) (end 36.5 67.56) (width 0.3) (layer "B.Cu") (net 3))
 (segment (start 36.5 66.56) (end 41.8 61.26) (width 0.3) (layer "B.Cu") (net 3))
 (segment (start 38.5 80.06) (end 36.5 78.06) (width 0.3) (layer "B.Cu") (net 3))
 (segment (start 47.04023 46.06) (end 49.04023 44.06) (width 0.3) (layer "B.Cu") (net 3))
 (segment (start 54 42.06) (end 63.5 51.56) (width 0.3) (layer "B.Cu") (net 3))
 (segment (start 41.8 61.26) (end 41.8 55.68) (width 0.3) (layer "B.Cu") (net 3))
 (segment (start 73.98 52.48) (end 75.08 52.48) (width 0.3) (layer "B.Cu") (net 3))
 (segment (start 35.5 71.06) (end 40.5 71.06) (width 0.5) (layer "F.Cu") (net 1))
 (via (at 40.5 71.06) (size 0.6) (drill 0.3) (layers "F.Cu" "B.Cu") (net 1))
 (via (at 35.5 71.06) (size 0.6) (drill 0.3) (layers "F.Cu" "B.Cu") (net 1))
 (segment (start 51.96 55.68) (end 55.58 52.06) (width 0.5) (layer "B.Cu") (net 1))
 (segment (start 40.62 71.06) (end 40.5 71.06) (width 0.5) (layer "B.Cu") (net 1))
 (segment (start 31.42 68.48) (end 34 71.06) (width 0.5) (layer "B.Cu") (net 1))
 (segment (start 50.38 67.56) (end 50.5 67.68) (width 0.5) (layer "B.Cu") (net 1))
 (segment (start 60.5 52.06) (end 71.1 62.66) (width 0.5) (layer "B.Cu") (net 1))
 (segment (start 44.12 67.56) (end 50.38 67.56) (width 0.5) (layer "B.Cu") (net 1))
 (segment (start 51.96 55.68) (end 50.5 57.14) (width 0.5) (layer "B.Cu") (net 1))
 (segment (start 71.12 62.64) (end 75.08 62.64) (width 0.5) (layer "B.Cu") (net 1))
 (segment (start 50.5 57.14) (end 50.5 67.68) (width 0.5) (layer "B.Cu") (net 1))
 (segment (start 31.42 67.56) (end 31.42 68.48) (width 0.5) (layer "B.Cu") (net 1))
 (segment (start 44.12 67.56) (end 40.62 71.06) (width 0.5) (layer "B.Cu") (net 1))
 (segment (start 34 71.06) (end 35.5 71.06) (width 0.5) (layer "B.Cu") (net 1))
 (segment (start 55.58 52.06) (end 60.5 52.06) (width 0.5) (layer "B.Cu") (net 1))
 (segment (start 71.1 62.66) (end 71.12 62.64) (width 0.5) (layer "B.Cu") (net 1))
 (segment (start 70.02 28.14) (end 71.08 27.08) (width 0.3) (layer "B.Cu") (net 13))
 (segment (start 71.08 27.08) (end 75.08 27.08) (width 0.3) (layer "B.Cu") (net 13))
 (segment (start 54.5 28.14) (end 70.02 28.14) (width 0.3) (layer "B.Cu") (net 13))
 (segment (start 70.02 30.68) (end 71.08 29.62) (width 0.3) (layer "B.Cu") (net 14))
 (segment (start 71.08 29.62) (end 75.08 29.62) (width 0.3) (layer "B.Cu") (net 14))
 (segment (start 54.5 30.68) (end 70.02 30.68) (width 0.3) (layer "B.Cu") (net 14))
 (segment (start 63.5 40.56) (end 63.5 37.56) (width 0.3) (layer "F.Cu") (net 16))
 (via (at 63.5 37.56) (size 0.6) (drill 0.3) (layers "F.Cu" "B.Cu") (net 16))
 (via (at 63.5 40.56) (size 0.6) (drill 0.3) (layers "F.Cu" "B.Cu") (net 16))
 (segment (start 54.5 35.76) (end 61.7 35.76) (width 0.3) (layer "B.Cu") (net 16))
 (segment (start 61.7 35.76) (end 63.5 37.56) (width 0.3) (layer "B.Cu") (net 16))
 (segment (start 69.48 55.02) (end 68.52 55.02) (width 0.3) (layer "B.Cu") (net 16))
 (segment (start 68.52 55.02) (end 63.5 50) (width 0.3) (layer "B.Cu") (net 16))
 (segment (start 63.5 40.56) (end 63.5 50) (width 0.3) (layer "B.Cu") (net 16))
 (segment (start 69.48 55.02) (end 75.08 55.02) (width 0.3) (layer "B.Cu") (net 16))
 (segment (start 64 31.56) (end 68.5 27.06) (width 0.3) (layer "F.Cu") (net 15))
 (via (at 64 31.56) (size 0.6) (drill 0.3) (layers "F.Cu" "B.Cu") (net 15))
 (via (at 68.5 27.06) (size 0.6) (drill 0.3) (layers "F.Cu" "B.Cu") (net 15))
 (segment (start 71.02 24.54) (end 75.08 24.54) (width 0.3) (layer "B.Cu") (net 15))
 (segment (start 68.5 27.06) (end 68.56 27.06) (width 0.3) (layer "B.Cu") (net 15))
 (segment (start 62.34 33.22) (end 54.5 33.22) (width 0.3) (layer "B.Cu") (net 15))
 (segment (start 68.5 27.06) (end 71.02 24.54) (width 0.3) (layer "B.Cu") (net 15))
 (segment (start 64 31.56) (end 62.34 33.22) (width 0.3) (layer "B.Cu") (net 15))
 (segment (start 71.08 32.16) (end 75.08 32.16) (width 0.3) (layer "B.Cu") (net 17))
 (segment (start 63.68 39.56) (end 71.08 32.16) (width 0.3) (layer "B.Cu") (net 17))
 (segment (start 31 38.56) (end 32 39.56) (width 0.3) (layer "B.Cu") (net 17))
 (segment (start 32 39.56) (end 63.68 39.56) (width 0.3) (layer "B.Cu") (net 17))
 (segment (start 27.46 35.02) (end 27.46 24.06) (width 0.3) (layer "B.Cu") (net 17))
 (segment (start 31 38.56) (end 27.46 35.02) (width 0.3) (layer "B.Cu") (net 17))
 (segment (start 33 91.06) (end 44.5 91.06) (width 0.3) (layer "B.Cu") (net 7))
 (segment (start 61.62 91.06) (end 44.5 91.06) (width 0.3) (layer "B.Cu") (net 7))
 (segment (start 25 83.06) (end 33 91.06) (width 0.3) (layer "B.Cu") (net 7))
 (segment (start 65.81 86.87) (end 61.62 91.06) (width 0.3) (layer "B.Cu") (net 7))
 (segment (start 44.5 91.06) (end 51.69 83.87) (width 0.3) (layer "B.Cu") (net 7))
 (segment (start 51.69 83.87) (end 51.69 79.56) (width 0.3) (layer "B.Cu") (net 7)))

